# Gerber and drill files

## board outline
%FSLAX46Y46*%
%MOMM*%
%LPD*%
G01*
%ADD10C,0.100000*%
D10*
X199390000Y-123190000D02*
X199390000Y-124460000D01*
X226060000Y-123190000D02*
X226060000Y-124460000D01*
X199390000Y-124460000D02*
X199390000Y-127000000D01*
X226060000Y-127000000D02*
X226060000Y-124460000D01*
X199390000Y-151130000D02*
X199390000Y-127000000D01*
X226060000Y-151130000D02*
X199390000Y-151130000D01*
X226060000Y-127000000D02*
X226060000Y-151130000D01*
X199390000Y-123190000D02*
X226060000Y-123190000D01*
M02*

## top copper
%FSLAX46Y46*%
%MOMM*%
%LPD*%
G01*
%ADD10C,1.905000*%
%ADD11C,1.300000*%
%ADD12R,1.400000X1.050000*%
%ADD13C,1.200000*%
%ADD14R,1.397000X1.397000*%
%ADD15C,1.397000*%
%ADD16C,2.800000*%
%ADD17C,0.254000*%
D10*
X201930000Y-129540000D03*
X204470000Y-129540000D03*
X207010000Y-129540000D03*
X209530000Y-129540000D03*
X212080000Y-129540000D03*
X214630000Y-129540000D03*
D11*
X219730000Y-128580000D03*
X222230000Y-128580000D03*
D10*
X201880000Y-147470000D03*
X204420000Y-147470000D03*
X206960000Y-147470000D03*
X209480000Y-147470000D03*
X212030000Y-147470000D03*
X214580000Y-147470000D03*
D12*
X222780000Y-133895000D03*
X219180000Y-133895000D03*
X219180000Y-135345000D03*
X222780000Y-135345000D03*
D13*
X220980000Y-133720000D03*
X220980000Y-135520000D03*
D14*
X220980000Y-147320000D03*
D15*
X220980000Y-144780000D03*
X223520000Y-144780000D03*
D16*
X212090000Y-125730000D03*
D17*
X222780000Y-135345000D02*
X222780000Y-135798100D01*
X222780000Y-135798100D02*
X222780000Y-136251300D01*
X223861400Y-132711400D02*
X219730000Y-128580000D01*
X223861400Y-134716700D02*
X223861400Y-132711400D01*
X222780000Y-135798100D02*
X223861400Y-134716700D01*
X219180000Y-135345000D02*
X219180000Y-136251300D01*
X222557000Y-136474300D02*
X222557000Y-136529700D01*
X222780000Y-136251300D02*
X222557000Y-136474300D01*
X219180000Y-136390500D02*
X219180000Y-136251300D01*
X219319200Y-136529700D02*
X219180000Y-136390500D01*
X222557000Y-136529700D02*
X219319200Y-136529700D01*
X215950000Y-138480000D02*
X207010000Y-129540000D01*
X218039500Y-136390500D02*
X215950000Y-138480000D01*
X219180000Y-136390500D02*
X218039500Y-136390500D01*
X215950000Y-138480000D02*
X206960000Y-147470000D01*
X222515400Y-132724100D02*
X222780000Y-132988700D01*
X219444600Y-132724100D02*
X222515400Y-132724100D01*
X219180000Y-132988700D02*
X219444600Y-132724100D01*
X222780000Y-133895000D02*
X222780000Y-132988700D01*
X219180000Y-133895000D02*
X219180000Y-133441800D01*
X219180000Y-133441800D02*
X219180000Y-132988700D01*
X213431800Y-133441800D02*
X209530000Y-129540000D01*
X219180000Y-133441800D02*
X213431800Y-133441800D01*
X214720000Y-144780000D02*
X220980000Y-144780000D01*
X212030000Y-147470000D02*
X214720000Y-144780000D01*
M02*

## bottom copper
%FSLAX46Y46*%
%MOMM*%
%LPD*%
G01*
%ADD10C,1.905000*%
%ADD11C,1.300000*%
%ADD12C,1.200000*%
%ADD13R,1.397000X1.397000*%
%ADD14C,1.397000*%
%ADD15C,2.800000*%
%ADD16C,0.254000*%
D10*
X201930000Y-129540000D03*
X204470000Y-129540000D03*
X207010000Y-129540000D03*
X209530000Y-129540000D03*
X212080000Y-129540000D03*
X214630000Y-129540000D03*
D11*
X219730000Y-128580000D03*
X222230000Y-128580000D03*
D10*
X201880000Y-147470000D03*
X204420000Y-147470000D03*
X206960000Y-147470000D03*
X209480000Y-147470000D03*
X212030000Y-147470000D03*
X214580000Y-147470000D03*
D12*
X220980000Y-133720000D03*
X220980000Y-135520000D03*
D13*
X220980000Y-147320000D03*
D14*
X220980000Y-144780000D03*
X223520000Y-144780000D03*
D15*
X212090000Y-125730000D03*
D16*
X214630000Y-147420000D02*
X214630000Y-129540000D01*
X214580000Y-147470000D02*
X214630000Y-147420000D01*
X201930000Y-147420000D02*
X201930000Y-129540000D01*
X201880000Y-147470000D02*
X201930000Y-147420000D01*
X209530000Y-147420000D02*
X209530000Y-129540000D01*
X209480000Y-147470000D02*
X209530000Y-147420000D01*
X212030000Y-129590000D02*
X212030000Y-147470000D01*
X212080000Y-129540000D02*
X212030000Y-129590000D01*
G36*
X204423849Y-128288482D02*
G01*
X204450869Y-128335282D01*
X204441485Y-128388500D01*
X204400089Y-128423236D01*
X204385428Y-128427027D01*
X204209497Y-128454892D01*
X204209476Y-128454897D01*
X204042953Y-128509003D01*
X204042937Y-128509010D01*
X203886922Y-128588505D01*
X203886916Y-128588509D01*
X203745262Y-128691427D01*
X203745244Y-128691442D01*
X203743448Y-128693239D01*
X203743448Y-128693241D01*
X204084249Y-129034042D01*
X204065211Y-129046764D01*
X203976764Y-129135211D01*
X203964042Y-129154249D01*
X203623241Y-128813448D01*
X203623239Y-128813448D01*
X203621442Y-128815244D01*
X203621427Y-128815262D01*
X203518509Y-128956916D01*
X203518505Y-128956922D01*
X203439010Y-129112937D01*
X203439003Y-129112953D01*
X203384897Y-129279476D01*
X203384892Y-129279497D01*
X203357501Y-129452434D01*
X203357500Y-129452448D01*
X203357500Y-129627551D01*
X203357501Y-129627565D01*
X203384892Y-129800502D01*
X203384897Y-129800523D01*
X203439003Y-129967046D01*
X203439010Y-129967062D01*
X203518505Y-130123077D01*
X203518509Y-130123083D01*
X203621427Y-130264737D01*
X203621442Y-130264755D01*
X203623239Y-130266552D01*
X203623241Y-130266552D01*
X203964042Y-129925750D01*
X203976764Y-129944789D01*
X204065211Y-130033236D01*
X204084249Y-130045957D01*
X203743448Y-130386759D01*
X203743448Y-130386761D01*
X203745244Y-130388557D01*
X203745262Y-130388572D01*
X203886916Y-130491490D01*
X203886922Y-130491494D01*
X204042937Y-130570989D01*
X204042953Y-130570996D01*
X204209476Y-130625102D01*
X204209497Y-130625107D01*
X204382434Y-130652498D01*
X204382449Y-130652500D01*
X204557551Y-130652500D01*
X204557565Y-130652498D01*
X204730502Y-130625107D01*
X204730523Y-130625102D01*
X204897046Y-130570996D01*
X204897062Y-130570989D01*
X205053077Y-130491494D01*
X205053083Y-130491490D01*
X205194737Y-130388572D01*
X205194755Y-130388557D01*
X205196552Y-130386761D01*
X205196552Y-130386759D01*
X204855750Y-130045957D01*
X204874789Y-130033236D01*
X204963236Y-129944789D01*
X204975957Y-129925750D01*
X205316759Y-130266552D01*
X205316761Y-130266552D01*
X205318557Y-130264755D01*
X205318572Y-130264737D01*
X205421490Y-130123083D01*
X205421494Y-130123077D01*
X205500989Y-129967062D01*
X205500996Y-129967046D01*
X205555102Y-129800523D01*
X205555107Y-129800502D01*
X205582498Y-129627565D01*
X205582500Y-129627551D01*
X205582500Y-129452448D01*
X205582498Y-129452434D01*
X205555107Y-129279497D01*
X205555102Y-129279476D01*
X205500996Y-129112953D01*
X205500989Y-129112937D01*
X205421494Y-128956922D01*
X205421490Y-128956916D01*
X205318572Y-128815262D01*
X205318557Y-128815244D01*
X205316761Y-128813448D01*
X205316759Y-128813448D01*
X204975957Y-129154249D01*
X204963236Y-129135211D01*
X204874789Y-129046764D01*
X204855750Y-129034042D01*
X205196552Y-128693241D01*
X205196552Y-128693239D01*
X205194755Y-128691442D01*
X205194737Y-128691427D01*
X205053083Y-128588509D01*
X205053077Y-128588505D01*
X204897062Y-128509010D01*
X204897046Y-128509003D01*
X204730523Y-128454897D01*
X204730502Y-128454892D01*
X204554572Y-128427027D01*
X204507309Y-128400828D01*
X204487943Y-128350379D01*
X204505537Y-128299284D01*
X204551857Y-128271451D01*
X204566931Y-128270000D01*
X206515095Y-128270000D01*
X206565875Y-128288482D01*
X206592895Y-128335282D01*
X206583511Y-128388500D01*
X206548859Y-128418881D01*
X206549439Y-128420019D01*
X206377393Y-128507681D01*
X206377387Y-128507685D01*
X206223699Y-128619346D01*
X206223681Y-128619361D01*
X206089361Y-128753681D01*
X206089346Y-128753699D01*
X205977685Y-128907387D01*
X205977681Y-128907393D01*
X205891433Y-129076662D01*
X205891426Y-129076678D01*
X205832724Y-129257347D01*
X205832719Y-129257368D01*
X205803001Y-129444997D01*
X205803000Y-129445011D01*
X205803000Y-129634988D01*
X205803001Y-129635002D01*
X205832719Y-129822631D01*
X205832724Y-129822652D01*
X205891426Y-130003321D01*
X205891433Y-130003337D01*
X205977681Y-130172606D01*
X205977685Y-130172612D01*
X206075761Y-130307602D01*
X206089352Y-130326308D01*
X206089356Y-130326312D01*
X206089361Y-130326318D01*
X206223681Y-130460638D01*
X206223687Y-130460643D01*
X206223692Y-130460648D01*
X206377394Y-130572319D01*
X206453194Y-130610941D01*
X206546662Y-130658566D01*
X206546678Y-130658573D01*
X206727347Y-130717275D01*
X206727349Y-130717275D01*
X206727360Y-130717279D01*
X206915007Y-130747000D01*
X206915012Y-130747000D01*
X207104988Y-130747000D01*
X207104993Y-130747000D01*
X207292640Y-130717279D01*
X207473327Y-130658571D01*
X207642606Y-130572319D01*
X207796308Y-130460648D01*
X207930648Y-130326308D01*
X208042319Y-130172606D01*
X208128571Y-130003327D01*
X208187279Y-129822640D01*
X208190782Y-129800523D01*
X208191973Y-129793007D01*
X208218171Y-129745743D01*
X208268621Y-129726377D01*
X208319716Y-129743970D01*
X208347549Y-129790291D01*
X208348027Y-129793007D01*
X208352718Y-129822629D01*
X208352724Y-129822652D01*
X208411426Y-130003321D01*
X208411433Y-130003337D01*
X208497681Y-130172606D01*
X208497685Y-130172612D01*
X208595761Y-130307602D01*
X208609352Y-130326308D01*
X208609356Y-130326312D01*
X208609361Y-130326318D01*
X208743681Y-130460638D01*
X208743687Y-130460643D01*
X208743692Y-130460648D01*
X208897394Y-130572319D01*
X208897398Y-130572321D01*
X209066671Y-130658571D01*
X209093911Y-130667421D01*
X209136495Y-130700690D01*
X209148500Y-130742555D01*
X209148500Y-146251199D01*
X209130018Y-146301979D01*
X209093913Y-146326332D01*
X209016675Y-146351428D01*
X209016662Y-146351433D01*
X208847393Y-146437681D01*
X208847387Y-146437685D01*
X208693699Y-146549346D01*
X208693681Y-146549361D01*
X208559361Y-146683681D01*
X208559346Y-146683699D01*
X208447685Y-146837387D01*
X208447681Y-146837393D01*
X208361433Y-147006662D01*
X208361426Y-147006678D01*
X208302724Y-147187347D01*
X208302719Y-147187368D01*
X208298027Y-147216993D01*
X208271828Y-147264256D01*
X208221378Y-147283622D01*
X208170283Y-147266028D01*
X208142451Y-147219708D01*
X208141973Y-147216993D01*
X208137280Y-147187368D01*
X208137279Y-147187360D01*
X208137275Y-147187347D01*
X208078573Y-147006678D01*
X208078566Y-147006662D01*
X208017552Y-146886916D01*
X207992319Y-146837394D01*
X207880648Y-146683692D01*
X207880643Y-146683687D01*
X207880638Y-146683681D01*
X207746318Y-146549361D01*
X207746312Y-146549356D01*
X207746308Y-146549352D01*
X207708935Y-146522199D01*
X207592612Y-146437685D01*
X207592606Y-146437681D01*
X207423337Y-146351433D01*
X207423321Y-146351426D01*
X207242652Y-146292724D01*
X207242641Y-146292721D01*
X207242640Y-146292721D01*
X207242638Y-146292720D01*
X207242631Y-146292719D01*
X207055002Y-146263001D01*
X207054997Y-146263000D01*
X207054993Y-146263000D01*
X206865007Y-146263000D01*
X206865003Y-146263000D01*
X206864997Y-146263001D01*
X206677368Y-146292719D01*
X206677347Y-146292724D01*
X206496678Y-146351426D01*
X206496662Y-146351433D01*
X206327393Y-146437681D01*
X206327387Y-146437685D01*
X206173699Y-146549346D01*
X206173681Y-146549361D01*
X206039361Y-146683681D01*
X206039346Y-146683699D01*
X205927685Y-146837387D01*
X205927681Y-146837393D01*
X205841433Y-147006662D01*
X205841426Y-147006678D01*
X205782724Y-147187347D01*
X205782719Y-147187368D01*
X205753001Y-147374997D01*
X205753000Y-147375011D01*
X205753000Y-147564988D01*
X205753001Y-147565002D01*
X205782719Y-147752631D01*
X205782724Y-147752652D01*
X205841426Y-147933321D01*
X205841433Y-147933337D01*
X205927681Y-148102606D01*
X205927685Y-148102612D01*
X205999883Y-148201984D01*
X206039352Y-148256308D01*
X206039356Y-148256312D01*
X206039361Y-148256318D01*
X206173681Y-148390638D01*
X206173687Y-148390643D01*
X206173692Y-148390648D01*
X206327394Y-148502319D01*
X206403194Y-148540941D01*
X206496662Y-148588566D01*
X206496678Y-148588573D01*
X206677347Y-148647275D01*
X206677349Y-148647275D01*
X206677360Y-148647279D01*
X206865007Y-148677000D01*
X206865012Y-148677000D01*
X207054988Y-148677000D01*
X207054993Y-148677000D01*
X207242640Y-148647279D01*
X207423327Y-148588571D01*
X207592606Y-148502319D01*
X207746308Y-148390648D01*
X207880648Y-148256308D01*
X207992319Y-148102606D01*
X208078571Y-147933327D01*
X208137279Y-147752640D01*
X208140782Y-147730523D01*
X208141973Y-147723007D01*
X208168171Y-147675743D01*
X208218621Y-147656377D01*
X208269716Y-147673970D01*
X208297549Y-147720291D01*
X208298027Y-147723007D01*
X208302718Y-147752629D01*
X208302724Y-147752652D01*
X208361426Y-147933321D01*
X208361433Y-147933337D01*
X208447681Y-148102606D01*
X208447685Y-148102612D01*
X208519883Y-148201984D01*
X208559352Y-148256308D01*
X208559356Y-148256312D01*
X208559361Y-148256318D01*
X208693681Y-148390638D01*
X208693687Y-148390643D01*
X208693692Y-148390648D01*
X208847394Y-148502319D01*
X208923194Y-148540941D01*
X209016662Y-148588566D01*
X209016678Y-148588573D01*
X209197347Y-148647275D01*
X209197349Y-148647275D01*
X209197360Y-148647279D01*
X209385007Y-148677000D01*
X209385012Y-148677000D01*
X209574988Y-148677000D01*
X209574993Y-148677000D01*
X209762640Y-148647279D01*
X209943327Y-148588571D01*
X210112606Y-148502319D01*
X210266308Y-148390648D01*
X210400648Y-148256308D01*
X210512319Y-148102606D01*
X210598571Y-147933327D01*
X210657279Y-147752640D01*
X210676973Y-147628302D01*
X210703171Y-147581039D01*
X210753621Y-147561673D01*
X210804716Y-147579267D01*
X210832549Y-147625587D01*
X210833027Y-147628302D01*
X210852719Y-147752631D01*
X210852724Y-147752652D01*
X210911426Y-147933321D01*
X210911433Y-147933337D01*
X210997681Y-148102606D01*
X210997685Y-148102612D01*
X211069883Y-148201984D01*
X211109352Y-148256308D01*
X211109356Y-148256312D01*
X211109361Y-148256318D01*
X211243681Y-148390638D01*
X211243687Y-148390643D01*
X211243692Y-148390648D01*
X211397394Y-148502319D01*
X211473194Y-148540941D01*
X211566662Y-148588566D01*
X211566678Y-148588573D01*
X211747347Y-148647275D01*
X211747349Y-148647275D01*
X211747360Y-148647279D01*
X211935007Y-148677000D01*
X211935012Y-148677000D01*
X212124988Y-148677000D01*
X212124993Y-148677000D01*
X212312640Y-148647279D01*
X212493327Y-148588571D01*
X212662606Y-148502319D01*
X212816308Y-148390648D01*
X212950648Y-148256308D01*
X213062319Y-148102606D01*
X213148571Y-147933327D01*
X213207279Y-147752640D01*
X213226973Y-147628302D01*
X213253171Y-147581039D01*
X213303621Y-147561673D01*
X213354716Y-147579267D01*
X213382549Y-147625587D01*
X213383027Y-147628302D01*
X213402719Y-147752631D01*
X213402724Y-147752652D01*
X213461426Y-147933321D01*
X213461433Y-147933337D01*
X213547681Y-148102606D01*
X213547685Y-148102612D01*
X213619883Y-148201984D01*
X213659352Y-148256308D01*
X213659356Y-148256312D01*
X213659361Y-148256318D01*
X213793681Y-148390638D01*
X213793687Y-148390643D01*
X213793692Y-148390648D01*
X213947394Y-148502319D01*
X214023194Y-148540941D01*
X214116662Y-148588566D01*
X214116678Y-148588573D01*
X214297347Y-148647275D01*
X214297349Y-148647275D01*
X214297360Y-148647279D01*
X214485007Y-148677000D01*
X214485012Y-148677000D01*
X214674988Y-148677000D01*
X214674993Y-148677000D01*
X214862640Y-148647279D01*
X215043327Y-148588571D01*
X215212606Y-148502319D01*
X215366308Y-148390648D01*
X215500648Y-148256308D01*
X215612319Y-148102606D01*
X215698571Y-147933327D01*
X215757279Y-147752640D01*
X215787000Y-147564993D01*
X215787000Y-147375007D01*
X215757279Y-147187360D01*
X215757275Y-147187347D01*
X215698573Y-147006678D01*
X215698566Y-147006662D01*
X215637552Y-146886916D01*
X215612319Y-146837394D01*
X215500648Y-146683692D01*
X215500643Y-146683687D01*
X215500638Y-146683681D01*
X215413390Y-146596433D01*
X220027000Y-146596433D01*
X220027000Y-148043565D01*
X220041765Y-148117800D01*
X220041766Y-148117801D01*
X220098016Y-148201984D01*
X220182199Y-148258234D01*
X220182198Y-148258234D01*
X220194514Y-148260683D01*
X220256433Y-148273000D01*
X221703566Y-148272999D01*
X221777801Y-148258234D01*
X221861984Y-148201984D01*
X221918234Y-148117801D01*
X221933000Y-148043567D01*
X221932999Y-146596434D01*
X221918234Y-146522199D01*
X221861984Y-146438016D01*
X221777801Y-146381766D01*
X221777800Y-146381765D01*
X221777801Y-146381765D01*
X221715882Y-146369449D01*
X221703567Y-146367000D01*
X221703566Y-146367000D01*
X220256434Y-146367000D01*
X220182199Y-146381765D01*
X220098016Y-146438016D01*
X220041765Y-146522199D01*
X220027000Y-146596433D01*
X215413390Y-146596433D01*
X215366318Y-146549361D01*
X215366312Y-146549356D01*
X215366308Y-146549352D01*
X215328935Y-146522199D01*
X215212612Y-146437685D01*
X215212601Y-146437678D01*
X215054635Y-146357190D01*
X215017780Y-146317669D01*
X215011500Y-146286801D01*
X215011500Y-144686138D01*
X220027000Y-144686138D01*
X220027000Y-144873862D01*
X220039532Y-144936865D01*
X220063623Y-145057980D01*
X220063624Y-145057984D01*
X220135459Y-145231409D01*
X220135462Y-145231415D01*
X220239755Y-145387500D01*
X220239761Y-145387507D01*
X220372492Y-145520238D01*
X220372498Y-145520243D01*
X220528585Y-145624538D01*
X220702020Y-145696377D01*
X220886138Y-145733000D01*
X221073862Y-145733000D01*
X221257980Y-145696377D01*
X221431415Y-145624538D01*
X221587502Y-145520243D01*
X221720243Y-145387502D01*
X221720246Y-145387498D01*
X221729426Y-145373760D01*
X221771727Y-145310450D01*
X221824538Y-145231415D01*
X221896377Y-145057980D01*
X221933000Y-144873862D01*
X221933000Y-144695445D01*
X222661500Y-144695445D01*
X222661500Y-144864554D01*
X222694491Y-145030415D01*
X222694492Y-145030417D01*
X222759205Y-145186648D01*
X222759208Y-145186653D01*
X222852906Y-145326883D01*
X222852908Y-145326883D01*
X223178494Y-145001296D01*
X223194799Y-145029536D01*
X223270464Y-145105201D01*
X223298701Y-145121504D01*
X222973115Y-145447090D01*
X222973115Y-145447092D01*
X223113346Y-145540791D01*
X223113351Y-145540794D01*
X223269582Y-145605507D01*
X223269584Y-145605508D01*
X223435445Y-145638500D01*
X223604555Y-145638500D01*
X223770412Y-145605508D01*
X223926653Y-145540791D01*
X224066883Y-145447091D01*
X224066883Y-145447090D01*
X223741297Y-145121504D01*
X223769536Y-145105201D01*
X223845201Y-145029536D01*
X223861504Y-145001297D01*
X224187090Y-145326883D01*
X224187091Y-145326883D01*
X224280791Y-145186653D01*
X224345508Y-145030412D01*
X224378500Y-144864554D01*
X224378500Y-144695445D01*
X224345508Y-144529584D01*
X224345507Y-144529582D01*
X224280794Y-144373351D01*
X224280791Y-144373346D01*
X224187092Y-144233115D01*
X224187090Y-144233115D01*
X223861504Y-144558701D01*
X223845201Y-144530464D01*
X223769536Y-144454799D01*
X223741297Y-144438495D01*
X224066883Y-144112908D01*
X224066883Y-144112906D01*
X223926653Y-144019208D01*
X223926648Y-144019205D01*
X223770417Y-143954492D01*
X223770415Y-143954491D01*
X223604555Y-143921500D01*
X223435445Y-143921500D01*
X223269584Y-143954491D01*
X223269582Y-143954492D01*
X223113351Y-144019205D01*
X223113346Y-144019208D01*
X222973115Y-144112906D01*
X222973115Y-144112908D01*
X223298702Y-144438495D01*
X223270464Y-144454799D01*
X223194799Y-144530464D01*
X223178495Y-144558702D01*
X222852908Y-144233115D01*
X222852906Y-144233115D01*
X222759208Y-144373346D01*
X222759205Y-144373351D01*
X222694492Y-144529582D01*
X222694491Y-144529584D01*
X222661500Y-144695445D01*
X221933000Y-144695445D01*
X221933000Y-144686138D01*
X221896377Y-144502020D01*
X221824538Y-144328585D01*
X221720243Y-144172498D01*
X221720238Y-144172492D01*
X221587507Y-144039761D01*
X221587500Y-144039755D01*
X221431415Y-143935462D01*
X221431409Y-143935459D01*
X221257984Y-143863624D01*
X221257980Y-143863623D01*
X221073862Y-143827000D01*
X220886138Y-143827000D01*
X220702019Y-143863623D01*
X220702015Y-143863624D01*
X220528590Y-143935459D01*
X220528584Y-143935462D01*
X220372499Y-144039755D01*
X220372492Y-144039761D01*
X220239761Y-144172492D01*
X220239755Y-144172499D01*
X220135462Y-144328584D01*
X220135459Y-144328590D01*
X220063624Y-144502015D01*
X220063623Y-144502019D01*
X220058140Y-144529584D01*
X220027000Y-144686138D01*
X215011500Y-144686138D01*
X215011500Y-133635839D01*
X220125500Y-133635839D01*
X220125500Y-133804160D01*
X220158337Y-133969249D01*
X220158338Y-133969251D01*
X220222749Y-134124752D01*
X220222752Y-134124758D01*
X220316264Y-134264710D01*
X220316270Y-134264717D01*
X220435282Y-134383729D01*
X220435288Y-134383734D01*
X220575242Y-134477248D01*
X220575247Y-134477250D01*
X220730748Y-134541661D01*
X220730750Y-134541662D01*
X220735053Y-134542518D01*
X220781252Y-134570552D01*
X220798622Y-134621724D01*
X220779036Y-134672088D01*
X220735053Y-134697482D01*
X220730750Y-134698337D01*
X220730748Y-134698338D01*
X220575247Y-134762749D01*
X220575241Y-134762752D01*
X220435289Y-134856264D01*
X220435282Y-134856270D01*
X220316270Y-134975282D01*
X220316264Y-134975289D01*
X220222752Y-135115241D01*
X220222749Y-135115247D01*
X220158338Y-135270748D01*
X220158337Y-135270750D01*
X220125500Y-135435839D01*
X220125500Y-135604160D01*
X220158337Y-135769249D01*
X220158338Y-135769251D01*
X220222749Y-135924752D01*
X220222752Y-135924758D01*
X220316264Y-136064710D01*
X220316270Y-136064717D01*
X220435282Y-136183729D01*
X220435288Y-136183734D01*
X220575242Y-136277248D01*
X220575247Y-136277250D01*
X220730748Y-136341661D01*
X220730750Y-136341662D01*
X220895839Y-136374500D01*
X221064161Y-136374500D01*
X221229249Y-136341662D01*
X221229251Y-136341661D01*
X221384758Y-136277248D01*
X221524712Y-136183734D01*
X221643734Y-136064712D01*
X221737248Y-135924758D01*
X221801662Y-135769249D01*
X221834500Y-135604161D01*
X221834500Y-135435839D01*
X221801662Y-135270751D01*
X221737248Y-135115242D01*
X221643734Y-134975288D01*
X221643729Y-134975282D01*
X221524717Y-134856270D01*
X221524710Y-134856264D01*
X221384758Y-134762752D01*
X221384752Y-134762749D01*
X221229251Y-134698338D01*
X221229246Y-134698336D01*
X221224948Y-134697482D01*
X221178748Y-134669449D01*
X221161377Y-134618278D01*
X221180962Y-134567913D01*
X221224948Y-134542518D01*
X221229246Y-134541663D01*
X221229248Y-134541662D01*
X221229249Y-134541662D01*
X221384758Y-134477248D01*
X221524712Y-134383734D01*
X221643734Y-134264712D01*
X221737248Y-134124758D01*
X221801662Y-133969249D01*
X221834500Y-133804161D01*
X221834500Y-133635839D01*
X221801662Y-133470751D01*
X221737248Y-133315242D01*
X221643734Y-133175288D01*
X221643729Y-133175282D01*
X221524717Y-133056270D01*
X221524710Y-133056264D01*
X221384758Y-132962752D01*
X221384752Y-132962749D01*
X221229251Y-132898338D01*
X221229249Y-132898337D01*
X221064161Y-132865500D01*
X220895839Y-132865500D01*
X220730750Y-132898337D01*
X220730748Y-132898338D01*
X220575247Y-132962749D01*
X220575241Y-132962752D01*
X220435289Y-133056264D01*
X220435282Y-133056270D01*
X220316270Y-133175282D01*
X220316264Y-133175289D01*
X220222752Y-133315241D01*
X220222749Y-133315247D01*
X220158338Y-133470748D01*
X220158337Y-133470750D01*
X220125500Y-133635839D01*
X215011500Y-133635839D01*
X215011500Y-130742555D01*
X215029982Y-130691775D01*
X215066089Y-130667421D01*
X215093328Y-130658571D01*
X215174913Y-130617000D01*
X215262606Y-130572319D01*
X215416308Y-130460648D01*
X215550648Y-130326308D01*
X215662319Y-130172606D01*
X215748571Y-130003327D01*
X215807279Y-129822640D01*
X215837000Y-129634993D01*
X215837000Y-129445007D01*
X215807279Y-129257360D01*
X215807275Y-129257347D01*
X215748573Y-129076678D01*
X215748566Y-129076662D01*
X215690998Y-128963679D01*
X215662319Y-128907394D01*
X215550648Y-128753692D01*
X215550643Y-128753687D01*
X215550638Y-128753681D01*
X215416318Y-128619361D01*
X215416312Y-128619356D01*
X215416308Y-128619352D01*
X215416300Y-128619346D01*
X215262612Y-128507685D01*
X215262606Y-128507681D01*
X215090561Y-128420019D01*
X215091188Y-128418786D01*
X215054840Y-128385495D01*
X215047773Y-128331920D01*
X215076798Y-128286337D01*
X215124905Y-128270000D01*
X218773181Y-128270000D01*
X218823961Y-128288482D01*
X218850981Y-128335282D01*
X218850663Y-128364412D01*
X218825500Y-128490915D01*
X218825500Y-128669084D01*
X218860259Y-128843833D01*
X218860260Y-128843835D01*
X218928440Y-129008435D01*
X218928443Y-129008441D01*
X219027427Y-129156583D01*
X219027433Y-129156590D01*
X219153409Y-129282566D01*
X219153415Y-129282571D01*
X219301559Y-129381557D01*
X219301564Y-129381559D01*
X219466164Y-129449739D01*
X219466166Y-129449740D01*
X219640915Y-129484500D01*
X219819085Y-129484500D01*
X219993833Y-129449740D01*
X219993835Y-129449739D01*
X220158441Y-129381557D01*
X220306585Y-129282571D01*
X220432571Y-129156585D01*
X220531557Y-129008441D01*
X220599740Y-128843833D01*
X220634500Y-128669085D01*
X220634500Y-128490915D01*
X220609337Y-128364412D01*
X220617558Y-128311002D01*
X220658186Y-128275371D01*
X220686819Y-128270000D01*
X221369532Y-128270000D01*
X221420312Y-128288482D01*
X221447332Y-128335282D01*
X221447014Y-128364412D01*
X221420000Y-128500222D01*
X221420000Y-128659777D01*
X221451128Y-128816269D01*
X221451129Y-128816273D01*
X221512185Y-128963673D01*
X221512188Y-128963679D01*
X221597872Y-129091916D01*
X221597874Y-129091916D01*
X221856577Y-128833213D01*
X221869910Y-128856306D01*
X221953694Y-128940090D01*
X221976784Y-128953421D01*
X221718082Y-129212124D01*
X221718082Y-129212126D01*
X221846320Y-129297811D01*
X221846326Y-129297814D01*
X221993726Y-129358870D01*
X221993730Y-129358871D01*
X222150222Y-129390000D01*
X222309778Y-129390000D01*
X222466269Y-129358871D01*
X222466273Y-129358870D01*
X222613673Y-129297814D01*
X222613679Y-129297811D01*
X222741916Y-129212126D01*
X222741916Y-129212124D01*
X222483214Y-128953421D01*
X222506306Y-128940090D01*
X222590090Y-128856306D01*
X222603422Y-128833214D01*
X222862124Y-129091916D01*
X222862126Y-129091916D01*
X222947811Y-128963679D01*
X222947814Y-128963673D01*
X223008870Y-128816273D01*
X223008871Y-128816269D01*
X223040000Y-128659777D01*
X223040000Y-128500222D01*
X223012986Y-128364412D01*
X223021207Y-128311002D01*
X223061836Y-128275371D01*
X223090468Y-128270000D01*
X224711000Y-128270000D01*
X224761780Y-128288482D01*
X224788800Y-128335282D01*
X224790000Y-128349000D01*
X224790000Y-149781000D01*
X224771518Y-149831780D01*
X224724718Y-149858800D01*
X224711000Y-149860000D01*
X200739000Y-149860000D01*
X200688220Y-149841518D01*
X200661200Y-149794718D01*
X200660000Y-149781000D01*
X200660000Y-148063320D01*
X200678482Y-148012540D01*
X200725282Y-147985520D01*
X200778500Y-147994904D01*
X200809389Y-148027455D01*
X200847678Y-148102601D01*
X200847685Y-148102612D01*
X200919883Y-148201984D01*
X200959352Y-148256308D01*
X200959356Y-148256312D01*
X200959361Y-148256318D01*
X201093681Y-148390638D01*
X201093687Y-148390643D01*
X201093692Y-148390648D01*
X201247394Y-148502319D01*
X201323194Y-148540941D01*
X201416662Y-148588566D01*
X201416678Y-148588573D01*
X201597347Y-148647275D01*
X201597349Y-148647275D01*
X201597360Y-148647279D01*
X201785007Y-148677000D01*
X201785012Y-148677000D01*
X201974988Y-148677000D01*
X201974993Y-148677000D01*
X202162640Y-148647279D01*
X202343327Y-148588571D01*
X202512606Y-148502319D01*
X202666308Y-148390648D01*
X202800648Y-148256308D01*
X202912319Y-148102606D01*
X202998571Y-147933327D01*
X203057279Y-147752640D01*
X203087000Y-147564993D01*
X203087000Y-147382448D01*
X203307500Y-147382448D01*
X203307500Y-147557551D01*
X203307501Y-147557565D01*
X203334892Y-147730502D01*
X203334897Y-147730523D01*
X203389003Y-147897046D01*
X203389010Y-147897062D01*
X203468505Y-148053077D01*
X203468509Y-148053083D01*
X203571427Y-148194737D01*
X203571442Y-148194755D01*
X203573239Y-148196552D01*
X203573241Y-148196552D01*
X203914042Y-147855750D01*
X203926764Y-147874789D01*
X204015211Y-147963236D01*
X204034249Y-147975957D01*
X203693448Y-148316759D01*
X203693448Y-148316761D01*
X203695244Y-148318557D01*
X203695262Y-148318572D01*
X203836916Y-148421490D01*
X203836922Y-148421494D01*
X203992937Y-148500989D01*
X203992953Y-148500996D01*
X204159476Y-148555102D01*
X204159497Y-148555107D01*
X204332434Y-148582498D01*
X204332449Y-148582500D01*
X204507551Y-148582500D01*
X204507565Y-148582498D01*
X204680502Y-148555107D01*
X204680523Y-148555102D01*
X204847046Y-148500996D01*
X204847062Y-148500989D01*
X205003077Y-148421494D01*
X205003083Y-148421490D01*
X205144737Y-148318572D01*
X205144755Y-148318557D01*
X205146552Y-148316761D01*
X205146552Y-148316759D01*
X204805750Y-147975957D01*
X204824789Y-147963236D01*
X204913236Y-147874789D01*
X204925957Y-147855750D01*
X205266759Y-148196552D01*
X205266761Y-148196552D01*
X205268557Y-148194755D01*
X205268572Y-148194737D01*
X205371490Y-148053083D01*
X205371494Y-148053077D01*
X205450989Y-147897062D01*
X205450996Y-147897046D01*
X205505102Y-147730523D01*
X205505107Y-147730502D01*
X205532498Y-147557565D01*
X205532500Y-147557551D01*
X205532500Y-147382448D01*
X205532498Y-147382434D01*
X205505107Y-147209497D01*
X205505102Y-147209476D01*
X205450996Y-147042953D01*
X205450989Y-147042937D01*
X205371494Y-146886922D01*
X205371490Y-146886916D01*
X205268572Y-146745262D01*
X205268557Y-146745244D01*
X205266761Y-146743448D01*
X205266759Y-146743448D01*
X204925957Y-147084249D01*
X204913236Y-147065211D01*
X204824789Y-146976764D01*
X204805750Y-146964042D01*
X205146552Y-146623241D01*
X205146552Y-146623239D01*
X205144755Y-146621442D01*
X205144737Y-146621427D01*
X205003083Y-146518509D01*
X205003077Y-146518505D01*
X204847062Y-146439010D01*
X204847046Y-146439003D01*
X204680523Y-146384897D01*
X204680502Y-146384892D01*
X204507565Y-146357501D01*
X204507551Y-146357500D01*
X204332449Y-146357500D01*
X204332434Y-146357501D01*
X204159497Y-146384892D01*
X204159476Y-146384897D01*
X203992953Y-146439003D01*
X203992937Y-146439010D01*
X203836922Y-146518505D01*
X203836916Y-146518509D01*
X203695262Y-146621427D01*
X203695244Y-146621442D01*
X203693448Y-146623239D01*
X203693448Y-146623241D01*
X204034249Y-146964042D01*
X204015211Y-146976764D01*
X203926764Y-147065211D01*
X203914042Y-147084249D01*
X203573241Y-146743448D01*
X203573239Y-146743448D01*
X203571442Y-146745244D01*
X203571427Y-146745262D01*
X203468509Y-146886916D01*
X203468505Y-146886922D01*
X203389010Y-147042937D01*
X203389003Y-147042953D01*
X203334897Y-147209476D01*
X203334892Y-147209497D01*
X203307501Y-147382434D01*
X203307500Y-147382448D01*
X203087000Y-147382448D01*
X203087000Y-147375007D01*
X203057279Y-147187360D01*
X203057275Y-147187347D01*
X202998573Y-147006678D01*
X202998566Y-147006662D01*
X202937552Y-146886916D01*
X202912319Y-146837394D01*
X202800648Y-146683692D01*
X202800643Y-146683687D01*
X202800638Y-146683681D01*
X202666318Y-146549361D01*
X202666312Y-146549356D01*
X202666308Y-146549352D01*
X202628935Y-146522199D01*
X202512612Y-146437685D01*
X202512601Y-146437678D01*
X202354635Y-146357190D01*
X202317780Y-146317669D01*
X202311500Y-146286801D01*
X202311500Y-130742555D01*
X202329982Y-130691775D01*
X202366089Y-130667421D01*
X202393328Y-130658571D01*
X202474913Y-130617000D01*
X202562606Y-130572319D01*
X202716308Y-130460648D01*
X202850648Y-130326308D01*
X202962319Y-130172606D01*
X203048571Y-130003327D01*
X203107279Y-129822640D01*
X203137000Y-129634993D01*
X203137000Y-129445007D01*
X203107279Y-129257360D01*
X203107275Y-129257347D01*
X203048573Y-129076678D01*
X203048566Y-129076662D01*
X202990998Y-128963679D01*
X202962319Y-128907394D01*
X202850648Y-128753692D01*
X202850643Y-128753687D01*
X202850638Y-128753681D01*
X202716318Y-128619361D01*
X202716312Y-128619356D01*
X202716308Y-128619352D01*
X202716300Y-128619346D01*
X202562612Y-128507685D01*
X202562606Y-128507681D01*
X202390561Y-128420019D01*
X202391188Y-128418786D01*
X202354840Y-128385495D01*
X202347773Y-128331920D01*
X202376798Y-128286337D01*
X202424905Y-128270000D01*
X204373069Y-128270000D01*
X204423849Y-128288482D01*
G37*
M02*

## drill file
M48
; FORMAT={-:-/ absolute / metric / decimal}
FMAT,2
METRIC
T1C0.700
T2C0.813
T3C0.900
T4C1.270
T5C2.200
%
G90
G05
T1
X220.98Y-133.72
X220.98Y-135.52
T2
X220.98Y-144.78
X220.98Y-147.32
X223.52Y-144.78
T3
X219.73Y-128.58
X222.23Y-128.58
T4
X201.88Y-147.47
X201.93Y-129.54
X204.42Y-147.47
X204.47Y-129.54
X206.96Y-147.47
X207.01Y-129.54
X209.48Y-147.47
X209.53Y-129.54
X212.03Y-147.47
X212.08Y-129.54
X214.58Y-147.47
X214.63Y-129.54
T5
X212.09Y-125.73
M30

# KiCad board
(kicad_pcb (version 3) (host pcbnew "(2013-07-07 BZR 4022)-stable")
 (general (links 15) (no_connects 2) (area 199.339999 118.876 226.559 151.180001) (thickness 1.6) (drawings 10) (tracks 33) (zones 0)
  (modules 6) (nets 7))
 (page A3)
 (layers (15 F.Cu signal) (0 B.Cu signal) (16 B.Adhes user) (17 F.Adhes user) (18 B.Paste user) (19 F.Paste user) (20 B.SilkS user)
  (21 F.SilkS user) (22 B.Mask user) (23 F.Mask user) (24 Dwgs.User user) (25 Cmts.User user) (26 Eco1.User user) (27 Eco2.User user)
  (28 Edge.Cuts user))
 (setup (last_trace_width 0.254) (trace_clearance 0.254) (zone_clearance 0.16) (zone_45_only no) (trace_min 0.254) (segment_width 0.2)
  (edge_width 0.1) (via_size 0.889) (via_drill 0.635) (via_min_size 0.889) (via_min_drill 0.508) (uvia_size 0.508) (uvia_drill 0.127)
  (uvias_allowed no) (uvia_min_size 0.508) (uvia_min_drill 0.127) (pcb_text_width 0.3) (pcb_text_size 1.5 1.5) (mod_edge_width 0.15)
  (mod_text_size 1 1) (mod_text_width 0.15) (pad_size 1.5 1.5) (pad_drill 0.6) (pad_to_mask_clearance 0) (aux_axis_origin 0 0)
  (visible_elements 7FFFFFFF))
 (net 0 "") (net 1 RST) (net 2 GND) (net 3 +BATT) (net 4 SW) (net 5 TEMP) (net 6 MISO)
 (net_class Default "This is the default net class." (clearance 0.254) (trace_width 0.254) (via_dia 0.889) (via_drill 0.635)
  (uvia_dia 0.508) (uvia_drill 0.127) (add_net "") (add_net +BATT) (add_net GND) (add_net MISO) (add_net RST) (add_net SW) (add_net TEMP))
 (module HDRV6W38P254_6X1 (layer F.Cu) (at 208.28 129.54)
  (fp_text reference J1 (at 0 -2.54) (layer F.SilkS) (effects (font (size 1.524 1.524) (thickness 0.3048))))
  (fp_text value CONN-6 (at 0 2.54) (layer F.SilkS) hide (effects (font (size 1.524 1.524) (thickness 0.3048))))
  (pad 1 thru_hole circle (at -6.35 0) (size 1.905 1.905) (drill 1.27) (layers *.Cu *.Mask F.SilkS) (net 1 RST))
  (pad 2 thru_hole circle (at -3.81 0) (size 1.905 1.905) (drill 1.27) (layers *.Cu *.Mask F.SilkS) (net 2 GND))
  (pad 3 thru_hole circle (at -1.27 0) (size 1.905 1.905) (drill 1.27) (layers *.Cu *.Mask F.SilkS) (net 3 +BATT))
  (pad 4 thru_hole circle (at 1.25 0) (size 1.905 1.905) (drill 1.27) (layers *.Cu *.Mask F.SilkS) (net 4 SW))
  (pad 5 thru_hole circle (at 3.8 0) (size 1.905 1.905) (drill 1.27) (layers *.Cu *.Mask F.SilkS) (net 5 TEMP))
  (pad 6 thru_hole circle (at 6.35 0) (size 1.905 1.905) (drill 1.27) (layers *.Cu *.Mask F.SilkS) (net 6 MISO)))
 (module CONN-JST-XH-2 (layer F.Cu) (at 220.98 119.38)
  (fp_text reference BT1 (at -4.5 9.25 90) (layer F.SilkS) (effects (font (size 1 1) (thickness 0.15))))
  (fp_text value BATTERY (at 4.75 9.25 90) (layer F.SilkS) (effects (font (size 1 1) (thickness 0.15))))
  (pad 1 thru_hole circle (at -1.25 9.2) (size 1.3 1.3) (drill 0.9) (layers *.Cu *.Mask F.SilkS) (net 3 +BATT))
  (pad 2 thru_hole circle (at 1.25 9.2) (size 1.3 1.3) (drill 0.9) (layers *.Cu *.Mask F.SilkS) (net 2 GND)))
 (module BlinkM (layer F.Cu) (at 208.28 140.97)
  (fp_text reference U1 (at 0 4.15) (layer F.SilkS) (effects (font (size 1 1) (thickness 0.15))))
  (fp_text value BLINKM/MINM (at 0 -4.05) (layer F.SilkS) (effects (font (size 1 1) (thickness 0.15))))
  (pad 1 thru_hole circle (at -6.4 6.5) (size 1.905 1.905) (drill 1.27) (layers *.Cu *.Mask F.SilkS) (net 1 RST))
  (pad 2 thru_hole circle (at -3.86 6.5) (size 1.905 1.905) (drill 1.27) (layers *.Cu *.Mask F.SilkS) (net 2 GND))
  (pad 3 thru_hole circle (at -1.32 6.5) (size 1.905 1.905) (drill 1.27) (layers *.Cu *.Mask F.SilkS) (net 3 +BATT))
  (pad 4 thru_hole circle (at 1.2 6.5) (size 1.905 1.905) (drill 1.27) (layers *.Cu *.Mask F.SilkS) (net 4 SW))
  (pad 5 thru_hole circle (at 3.75 6.5) (size 1.905 1.905) (drill 1.27) (layers *.Cu *.Mask F.SilkS) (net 5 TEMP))
  (pad 6 thru_hole circle (at 6.3 6.5) (size 1.905 1.905) (drill 1.27) (layers *.Cu *.Mask F.SilkS) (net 6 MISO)))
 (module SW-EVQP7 (layer F.Cu) (at 220.98 134.62)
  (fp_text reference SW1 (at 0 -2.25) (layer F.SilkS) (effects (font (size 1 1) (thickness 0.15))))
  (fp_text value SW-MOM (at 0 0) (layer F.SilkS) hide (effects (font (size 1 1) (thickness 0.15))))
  (pad 1 smd rect (at 1.8 -0.725) (size 1.4 1.05) (layers F.Cu F.Paste F.Mask) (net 4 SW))
  (pad 1 smd rect (at -1.8 -0.725) (size 1.4 1.05) (layers F.Cu F.Paste F.Mask) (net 4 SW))
  (pad 2 smd rect (at -1.8 0.725) (size 1.4 1.05) (layers F.Cu F.Paste F.Mask) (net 3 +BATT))
  (pad 2 smd rect (at 1.8 0.725) (size 1.4 1.05) (layers F.Cu F.Paste F.Mask) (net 3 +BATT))
  (pad "" thru_hole circle (at 0 -0.9) (size 1.2 1.2) (drill 0.7) (layers *.Cu *.Mask F.SilkS))
  (pad "" thru_hole circle (at 0 0.9) (size 1.2 1.2) (drill 0.7) (layers *.Cu *.Mask F.SilkS)))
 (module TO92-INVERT (layer F.Cu) (at 222.25 146.05)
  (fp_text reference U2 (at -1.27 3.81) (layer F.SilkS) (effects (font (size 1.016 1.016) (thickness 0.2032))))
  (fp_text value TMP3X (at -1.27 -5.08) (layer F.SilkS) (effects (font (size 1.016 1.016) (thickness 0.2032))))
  (pad 1 thru_hole rect (at -1.27 1.27) (size 1.397 1.397) (drill 0.8128) (layers *.Cu *.Mask F.SilkS) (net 3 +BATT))
  (pad 2 thru_hole circle (at -1.27 -1.27) (size 1.397 1.397) (drill 0.8128) (layers *.Cu *.Mask F.SilkS) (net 5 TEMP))
  (pad 3 thru_hole circle (at 1.27 -1.27) (size 1.397 1.397) (drill 0.8128) (layers *.Cu *.Mask F.SilkS) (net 2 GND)))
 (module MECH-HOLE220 (layer F.Cu) (at 212.09 125.73)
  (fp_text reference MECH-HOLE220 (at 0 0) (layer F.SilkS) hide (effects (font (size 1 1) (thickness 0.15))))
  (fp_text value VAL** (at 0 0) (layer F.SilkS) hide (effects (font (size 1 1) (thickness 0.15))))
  (pad "" thru_hole circle (at 0 0) (size 2.8 2.8) (drill 2.2) (layers *.Cu *.Mask F.SilkS)))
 (gr_line (start 199.39 123.19) (end 199.39 124.46) (angle 90) (layer Edge.Cuts) (width 0.1))
 (gr_line (start 226.06 123.19) (end 226.06 124.46) (angle 90) (layer Edge.Cuts) (width 0.1))
 (gr_line (start 199.39 124.46) (end 199.39 127) (angle 90) (layer Edge.Cuts) (width 0.1))
 (gr_line (start 226.06 127) (end 226.06 124.46) (angle 90) (layer Edge.Cuts) (width 0.1))
 (gr_line (start 199.39 151.13) (end 199.39 127) (angle 90) (layer Edge.Cuts) (width 0.1))
 (gr_line (start 226.06 151.13) (end 199.39 151.13) (angle 90) (layer Edge.Cuts) (width 0.1))
 (gr_line (start 226.06 127) (end 226.06 151.13) (angle 90) (layer Edge.Cuts) (width 0.1))
 (gr_line (start 199.39 123.19) (end 226.06 123.19) (angle 90) (layer Edge.Cuts) (width 0.1))
 (segment (start 222.78 135.345) (end 222.78 135.7981) (width 0.254) (layer F.Cu) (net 3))
 (segment (start 222.78 135.7981) (end 222.78 136.2513) (width 0.254) (layer F.Cu) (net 3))
 (segment (start 223.8614 132.7114) (end 219.73 128.58) (width 0.254) (layer F.Cu) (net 3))
 (segment (start 223.8614 134.7167) (end 223.8614 132.7114) (width 0.254) (layer F.Cu) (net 3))
 (segment (start 222.78 135.7981) (end 223.8614 134.7167) (width 0.254) (layer F.Cu) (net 3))
 (segment (start 219.18 135.345) (end 219.18 136.2513) (width 0.254) (layer F.Cu) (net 3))
 (segment (start 222.557 136.4743) (end 222.557 136.5297) (width 0.254) (layer F.Cu) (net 3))
 (segment (start 222.78 136.2513) (end 222.557 136.4743) (width 0.254) (layer F.Cu) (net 3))
 (segment (start 219.18 136.3905) (end 219.18 136.2513) (width 0.254) (layer F.Cu) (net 3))
 (segment (start 219.3192 136.5297) (end 219.18 136.3905) (width 0.254) (layer F.Cu) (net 3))
 (segment (start 222.557 136.5297) (end 219.3192 136.5297) (width 0.254) (layer F.Cu) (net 3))
 (segment (start 215.95 138.48) (end 207.01 129.54) (width 0.254) (layer F.Cu) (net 3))
 (segment (start 218.0395 136.3905) (end 215.95 138.48) (width 0.254) (layer F.Cu) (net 3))
 (segment (start 219.18 136.3905) (end 218.0395 136.3905) (width 0.254) (layer F.Cu) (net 3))
 (segment (start 215.95 138.48) (end 206.96 147.47) (width 0.254) (layer F.Cu) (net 3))
 (segment (start 214.63 147.42) (end 214.63 129.54) (width 0.254) (layer B.Cu) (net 6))
 (segment (start 214.58 147.47) (end 214.63 147.42) (width 0.254) (layer B.Cu) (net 6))
 (segment (start 201.93 147.42) (end 201.93 129.54) (width 0.254) (layer B.Cu) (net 1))
 (segment (start 201.88 147.47) (end 201.93 147.42) (width 0.254) (layer B.Cu) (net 1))
 (segment (start 222.5154 132.7241) (end 222.78 132.9887) (width 0.254) (layer F.Cu) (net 4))
 (segment (start 219.4446 132.7241) (end 222.5154 132.7241) (width 0.254) (layer F.Cu) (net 4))
 (segment (start 219.18 132.9887) (end 219.4446 132.7241) (width 0.254) (layer F.Cu) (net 4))
 (segment (start 222.78 133.895) (end 222.78 132.9887) (width 0.254) (layer F.Cu) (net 4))
 (segment (start 219.18 133.895) (end 219.18 133.4418) (width 0.254) (layer F.Cu) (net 4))
 (segment (start 219.18 133.4418) (end 219.18 132.9887) (width 0.254) (layer F.Cu) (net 4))
 (segment (start 213.4318 133.4418) (end 209.53 129.54) (width 0.254) (layer F.Cu) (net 4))
 (segment (start 219.18 133.4418) (end 213.4318 133.4418) (width 0.254) (layer F.Cu) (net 4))
 (segment (start 209.53 147.42) (end 209.53 129.54) (width 0.254) (layer B.Cu) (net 4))
 (segment (start 209.48 147.47) (end 209.53 147.42) (width 0.254) (layer B.Cu) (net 4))
 (segment (start 214.72 144.78) (end 220.98 144.78) (width 0.254) (layer F.Cu) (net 5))
 (segment (start 212.03 147.47) (end 214.72 144.78) (width 0.254) (layer F.Cu) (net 5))
 (segment (start 212.03 129.59) (end 212.03 147.47) (width 0.254) (layer B.Cu) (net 5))
 (segment (start 212.08 129.54) (end 212.03 129.59) (width 0.254) (layer B.Cu) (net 5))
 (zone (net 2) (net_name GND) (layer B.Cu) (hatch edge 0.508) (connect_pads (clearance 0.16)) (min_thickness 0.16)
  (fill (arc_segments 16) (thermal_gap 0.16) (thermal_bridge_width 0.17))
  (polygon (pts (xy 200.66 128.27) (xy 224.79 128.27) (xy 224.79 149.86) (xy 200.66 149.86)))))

